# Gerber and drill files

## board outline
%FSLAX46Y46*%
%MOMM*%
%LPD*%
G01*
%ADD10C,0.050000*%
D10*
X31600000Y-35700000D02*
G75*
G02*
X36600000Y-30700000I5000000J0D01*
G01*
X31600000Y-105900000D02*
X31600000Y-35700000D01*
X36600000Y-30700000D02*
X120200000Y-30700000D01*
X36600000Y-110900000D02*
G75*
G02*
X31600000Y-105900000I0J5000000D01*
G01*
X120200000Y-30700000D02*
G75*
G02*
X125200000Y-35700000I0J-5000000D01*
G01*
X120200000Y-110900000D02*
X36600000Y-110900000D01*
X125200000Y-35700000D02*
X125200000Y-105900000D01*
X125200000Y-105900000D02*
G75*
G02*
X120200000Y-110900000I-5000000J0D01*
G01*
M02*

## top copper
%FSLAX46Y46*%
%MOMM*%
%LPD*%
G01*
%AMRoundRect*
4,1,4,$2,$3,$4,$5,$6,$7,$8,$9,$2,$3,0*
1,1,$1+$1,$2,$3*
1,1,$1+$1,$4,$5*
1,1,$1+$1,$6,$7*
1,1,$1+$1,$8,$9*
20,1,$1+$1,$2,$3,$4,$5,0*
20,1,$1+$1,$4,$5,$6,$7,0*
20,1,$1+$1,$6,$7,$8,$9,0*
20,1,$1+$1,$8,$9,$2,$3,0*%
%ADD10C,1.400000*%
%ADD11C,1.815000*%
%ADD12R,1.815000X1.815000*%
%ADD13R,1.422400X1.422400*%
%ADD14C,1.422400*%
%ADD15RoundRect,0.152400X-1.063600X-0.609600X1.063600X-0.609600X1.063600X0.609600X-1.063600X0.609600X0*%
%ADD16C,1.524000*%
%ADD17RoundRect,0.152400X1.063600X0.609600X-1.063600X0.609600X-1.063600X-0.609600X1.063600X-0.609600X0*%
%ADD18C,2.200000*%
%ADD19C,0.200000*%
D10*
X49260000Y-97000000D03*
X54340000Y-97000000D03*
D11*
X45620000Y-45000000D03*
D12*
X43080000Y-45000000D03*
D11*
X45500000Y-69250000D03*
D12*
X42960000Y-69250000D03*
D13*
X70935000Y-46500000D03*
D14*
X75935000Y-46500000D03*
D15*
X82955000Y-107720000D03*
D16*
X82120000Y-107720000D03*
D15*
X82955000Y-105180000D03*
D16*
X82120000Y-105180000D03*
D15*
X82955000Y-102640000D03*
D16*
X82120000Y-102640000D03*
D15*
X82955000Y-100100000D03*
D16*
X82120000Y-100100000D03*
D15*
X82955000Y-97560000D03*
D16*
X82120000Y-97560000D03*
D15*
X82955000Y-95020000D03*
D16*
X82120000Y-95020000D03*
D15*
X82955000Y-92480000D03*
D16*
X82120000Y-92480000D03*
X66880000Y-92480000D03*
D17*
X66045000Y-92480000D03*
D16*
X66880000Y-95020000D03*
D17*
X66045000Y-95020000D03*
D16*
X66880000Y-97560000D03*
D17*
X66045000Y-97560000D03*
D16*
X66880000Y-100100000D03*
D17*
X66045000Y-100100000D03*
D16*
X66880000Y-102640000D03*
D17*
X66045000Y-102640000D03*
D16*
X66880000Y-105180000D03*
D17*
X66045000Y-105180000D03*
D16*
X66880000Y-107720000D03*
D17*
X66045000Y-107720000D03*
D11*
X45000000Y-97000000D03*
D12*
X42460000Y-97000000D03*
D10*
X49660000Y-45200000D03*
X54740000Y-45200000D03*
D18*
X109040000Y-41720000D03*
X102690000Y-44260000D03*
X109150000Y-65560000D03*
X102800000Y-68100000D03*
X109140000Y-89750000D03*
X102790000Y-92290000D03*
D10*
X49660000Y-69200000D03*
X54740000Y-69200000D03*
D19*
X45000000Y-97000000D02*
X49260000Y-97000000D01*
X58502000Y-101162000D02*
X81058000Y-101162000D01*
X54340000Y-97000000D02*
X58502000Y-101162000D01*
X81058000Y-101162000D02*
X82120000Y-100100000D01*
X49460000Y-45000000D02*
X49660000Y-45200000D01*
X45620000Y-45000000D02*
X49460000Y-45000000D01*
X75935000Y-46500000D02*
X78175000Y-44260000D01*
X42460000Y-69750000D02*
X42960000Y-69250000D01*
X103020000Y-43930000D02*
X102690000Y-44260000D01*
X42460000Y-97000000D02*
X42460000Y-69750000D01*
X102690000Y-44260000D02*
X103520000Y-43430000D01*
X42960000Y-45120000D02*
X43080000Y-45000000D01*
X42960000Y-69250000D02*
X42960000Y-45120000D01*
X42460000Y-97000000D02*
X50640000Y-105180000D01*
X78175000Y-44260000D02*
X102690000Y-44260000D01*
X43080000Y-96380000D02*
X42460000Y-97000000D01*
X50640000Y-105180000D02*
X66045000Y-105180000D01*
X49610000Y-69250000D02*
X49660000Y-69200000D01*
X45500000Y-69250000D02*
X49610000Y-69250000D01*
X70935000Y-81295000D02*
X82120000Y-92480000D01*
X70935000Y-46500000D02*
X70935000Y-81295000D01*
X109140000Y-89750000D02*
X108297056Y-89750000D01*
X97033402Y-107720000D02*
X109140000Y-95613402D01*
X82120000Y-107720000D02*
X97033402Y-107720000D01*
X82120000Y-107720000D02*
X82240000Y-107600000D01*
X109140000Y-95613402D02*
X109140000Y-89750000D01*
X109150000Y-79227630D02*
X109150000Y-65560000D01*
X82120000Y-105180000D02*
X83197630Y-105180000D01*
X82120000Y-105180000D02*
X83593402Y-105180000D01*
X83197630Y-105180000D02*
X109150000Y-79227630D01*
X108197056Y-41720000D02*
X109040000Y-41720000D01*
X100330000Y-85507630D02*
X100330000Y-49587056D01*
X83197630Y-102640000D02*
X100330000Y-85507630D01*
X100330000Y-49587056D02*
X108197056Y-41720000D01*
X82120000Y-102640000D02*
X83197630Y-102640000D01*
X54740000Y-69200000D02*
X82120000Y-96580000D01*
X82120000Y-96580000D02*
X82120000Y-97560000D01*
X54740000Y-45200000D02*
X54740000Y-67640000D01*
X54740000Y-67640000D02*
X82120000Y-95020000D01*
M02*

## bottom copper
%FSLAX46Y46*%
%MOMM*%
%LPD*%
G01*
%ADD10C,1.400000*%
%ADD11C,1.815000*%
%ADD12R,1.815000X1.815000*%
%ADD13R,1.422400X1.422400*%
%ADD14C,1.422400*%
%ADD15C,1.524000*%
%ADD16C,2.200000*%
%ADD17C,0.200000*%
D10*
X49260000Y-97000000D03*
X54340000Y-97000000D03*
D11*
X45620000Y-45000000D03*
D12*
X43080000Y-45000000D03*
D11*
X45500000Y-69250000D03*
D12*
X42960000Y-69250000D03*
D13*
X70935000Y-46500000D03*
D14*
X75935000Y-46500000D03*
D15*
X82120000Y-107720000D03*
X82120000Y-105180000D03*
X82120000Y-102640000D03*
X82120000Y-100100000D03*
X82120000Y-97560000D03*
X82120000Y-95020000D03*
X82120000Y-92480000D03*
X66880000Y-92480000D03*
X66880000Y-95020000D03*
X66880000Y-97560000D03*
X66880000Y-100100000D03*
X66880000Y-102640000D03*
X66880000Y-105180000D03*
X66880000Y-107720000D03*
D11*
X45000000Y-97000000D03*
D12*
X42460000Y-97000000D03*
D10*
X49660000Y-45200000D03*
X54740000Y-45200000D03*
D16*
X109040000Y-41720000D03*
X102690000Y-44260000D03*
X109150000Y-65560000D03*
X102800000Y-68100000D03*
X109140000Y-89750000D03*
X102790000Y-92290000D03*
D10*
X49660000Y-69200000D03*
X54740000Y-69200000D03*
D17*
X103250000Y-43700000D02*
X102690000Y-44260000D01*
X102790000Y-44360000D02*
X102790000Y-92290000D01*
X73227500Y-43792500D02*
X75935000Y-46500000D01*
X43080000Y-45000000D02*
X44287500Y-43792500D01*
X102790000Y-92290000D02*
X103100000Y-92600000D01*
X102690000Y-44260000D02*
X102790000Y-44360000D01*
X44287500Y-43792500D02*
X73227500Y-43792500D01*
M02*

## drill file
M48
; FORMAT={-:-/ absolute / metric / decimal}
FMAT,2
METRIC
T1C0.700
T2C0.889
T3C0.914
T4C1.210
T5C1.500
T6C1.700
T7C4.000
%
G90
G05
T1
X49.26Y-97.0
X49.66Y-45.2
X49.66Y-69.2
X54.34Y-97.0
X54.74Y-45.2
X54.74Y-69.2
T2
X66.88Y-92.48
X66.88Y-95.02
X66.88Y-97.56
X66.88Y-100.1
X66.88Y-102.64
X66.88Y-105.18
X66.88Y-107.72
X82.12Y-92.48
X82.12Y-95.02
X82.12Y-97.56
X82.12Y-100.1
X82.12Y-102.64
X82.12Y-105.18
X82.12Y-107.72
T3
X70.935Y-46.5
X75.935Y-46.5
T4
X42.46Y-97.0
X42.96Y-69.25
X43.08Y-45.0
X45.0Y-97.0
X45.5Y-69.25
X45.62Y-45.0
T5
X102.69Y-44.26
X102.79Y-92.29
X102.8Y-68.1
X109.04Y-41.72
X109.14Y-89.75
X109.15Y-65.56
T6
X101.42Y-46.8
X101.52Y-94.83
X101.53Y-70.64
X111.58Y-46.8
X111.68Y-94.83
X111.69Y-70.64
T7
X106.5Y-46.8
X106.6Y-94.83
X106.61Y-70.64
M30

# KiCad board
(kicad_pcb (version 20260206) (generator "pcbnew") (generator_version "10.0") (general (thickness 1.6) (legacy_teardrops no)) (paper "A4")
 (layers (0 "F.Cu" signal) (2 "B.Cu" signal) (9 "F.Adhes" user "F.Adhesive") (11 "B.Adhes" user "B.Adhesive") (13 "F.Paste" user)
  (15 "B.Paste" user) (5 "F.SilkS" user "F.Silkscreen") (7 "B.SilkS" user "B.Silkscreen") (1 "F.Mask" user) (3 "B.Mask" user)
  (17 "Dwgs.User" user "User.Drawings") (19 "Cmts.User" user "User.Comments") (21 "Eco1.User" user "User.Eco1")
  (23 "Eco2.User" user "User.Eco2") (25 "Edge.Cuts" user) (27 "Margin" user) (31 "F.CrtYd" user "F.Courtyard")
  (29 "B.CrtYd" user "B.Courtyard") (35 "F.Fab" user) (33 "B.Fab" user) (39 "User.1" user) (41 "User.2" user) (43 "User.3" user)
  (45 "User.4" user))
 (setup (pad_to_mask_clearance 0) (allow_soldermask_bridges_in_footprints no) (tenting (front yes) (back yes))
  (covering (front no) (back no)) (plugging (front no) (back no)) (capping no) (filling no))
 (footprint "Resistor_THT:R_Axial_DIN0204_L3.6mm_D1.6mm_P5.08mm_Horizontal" (layer "F.Cu") (at 49.26 97)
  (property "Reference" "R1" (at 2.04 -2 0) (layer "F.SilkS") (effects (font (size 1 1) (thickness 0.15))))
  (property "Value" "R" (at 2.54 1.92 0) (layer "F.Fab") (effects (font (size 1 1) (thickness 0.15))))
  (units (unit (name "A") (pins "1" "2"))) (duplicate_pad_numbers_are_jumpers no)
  (pad "1" thru_hole circle (at 0 0) (size 1.4 1.4) (drill 0.7) (layers "*.Cu" "*.Mask") (remove_unused_layers no) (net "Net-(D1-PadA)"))
  (pad "2" thru_hole circle (at 5.08 0) (size 1.4 1.4) (drill 0.7) (layers "*.Cu" "*.Mask") (remove_unused_layers no) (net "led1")))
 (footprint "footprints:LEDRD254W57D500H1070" (layer "F.Cu") (at 44.35 45)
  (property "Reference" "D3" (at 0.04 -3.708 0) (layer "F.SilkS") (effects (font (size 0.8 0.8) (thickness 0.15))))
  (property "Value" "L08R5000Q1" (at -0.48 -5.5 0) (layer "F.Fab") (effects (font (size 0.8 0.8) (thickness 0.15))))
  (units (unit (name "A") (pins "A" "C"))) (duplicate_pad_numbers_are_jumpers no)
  (pad "A" thru_hole circle (at 1.27 0) (size 1.815 1.815) (drill 1.21) (layers "*.Cu" "*.Mask") (remove_unused_layers no)
   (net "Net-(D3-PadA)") (solder_mask_margin 0.102))
  (pad "C" thru_hole rect (at -1.27 0) (size 1.815 1.815) (drill 1.21) (layers "*.Cu" "*.Mask") (remove_unused_layers no) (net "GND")
   (solder_mask_margin 0.102)))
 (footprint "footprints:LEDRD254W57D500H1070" (layer "F.Cu") (at 44.23 69.25)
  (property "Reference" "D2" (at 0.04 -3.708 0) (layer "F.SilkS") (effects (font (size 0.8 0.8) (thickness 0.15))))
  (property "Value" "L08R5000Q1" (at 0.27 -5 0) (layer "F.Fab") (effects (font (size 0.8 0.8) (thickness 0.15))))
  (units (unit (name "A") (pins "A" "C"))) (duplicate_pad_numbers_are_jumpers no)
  (pad "A" thru_hole circle (at 1.27 0) (size 1.815 1.815) (drill 1.21) (layers "*.Cu" "*.Mask") (remove_unused_layers no)
   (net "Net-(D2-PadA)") (solder_mask_margin 0.102))
  (pad "C" thru_hole rect (at -1.27 0) (size 1.815 1.815) (drill 1.21) (layers "*.Cu" "*.Mask") (remove_unused_layers no) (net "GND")
   (solder_mask_margin 0.102)))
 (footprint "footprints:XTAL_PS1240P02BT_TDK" (layer "F.Cu") (at 70.935 46.5)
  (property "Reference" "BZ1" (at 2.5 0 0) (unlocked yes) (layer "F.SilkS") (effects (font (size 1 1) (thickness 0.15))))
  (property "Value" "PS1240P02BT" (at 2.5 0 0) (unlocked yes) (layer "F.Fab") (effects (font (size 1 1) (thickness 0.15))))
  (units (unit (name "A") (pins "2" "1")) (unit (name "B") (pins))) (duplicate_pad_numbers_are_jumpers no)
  (pad "1" thru_hole rect (at 0 0) (size 1.4224 1.4224) (drill 0.9144) (layers "*.Cu" "*.Mask") (remove_unused_layers no) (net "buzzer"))
  (pad "2" thru_hole circle (at 5 0) (size 1.4224 1.4224) (drill 0.9144) (layers "*.Cu" "*.Mask") (remove_unused_layers no) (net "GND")))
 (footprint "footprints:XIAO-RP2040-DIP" (layer "F.Cu") (at 74.5 100.1 -90)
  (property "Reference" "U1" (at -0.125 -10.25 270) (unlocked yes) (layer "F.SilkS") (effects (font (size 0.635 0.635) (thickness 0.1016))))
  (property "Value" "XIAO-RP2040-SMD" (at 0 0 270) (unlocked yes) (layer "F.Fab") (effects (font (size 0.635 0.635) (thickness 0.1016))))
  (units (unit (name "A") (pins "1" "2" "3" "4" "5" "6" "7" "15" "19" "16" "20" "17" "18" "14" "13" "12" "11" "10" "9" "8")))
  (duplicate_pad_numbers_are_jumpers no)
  (pad "1" smd roundrect (at 7.62 -8.455) (size 2.432 1.524) (layers "F.Cu" "F.Mask") (roundrect_rratio 0.1) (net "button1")
   (thermal_bridge_angle 45))
  (pad "1" thru_hole circle (at 7.62 -7.62) (size 1.524 1.524) (drill 0.889) (layers "*.Cu" "*.Mask") (remove_unused_layers no)
   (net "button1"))
  (pad "2" smd roundrect (at 5.08 -8.455) (size 2.432 1.524) (layers "F.Cu" "F.Mask") (roundrect_rratio 0.1) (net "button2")
   (thermal_bridge_angle 45))
  (pad "2" thru_hole circle (at 5.08 -7.62) (size 1.524 1.524) (drill 0.889) (layers "*.Cu" "*.Mask") (remove_unused_layers no)
   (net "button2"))
  (pad "3" smd roundrect (at 2.54 -8.455) (size 2.432 1.524) (layers "F.Cu" "F.Mask") (roundrect_rratio 0.1) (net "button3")
   (thermal_bridge_angle 45))
  (pad "3" thru_hole circle (at 2.54 -7.62) (size 1.524 1.524) (drill 0.889) (layers "*.Cu" "*.Mask") (remove_unused_layers no)
   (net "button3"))
  (pad "4" smd roundrect (at 0 -8.455) (size 2.432 1.524) (layers "F.Cu" "F.Mask") (roundrect_rratio 0.1) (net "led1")
   (thermal_bridge_angle 45))
  (pad "4" thru_hole circle (at 0 -7.62) (size 1.524 1.524) (drill 0.889) (layers "*.Cu" "*.Mask") (remove_unused_layers no) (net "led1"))
  (pad "5" smd roundrect (at -2.54 -8.455) (size 2.432 1.524) (layers "F.Cu" "F.Mask") (roundrect_rratio 0.1) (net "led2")
   (thermal_bridge_angle 45))
  (pad "5" thru_hole circle (at -2.54 -7.62) (size 1.524 1.524) (drill 0.889) (layers "*.Cu" "*.Mask") (remove_unused_layers no)
   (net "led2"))
  (pad "6" smd roundrect (at -5.08 -8.455) (size 2.432 1.524) (layers "F.Cu" "F.Mask") (roundrect_rratio 0.1) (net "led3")
   (thermal_bridge_angle 45))
  (pad "6" thru_hole circle (at -5.08 -7.62) (size 1.524 1.524) (drill 0.889) (layers "*.Cu" "*.Mask") (remove_unused_layers no)
   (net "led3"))
  (pad "7" smd roundrect (at -7.62 -8.455) (size 2.432 1.524) (layers "F.Cu" "F.Mask") (roundrect_rratio 0.1) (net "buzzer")
   (thermal_bridge_angle 45))
  (pad "7" thru_hole circle (at -7.62 -7.62) (size 1.524 1.524) (drill 0.889) (layers "*.Cu" "*.Mask") (remove_unused_layers no)
   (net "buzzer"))
  (pad "8" thru_hole circle (at -7.62 7.62 180) (size 1.524 1.524) (drill 0.889) (layers "*.Cu" "*.Mask") (remove_unused_layers no)
   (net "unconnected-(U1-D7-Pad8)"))
  (pad "8" smd roundrect (at -7.62 8.455 180) (size 2.432 1.524) (layers "F.Cu" "F.Mask") (roundrect_rratio 0.1)
   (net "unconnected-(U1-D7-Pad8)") (thermal_bridge_angle 45))
  (pad "9" thru_hole circle (at -5.08 7.62 180) (size 1.524 1.524) (drill 0.889) (layers "*.Cu" "*.Mask") (remove_unused_layers no)
   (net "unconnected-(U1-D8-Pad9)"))
  (pad "9" smd roundrect (at -5.08 8.455 180) (size 2.432 1.524) (layers "F.Cu" "F.Mask") (roundrect_rratio 0.1)
   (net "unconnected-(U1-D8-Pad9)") (thermal_bridge_angle 45))
  (pad "10" thru_hole circle (at -2.54 7.62 180) (size 1.524 1.524) (drill 0.889) (layers "*.Cu" "*.Mask") (remove_unused_layers no)
   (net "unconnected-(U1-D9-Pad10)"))
  (pad "10" smd roundrect (at -2.54 8.455 180) (size 2.432 1.524) (layers "F.Cu" "F.Mask") (roundrect_rratio 0.1)
   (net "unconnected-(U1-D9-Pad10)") (thermal_bridge_angle 45))
  (pad "11" thru_hole circle (at 0 7.62 180) (size 1.524 1.524) (drill 0.889) (layers "*.Cu" "*.Mask") (remove_unused_layers no)
   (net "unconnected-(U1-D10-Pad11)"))
  (pad "11" smd roundrect (at 0 8.455 180) (size 2.432 1.524) (layers "F.Cu" "F.Mask") (roundrect_rratio 0.1)
   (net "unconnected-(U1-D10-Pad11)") (thermal_bridge_angle 45))
  (pad "12" thru_hole circle (at 2.54 7.62 180) (size 1.524 1.524) (drill 0.889) (layers "*.Cu" "*.Mask") (remove_unused_layers no)
   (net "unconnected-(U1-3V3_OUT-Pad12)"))
  (pad "12" smd roundrect (at 2.54 8.455 180) (size 2.432 1.524) (layers "F.Cu" "F.Mask") (roundrect_rratio 0.1)
   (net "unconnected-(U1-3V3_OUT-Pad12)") (thermal_bridge_angle 45))
  (pad "13" thru_hole circle (at 5.08 7.62 180) (size 1.524 1.524) (drill 0.889) (layers "*.Cu" "*.Mask") (remove_unused_layers no)
   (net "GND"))
  (pad "13" smd roundrect (at 5.08 8.455 180) (size 2.432 1.524) (layers "F.Cu" "F.Mask") (roundrect_rratio 0.1) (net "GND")
   (thermal_bridge_angle 45))
  (pad "14" thru_hole circle (at 7.62 7.62 180) (size 1.524 1.524) (drill 0.889) (layers "*.Cu" "*.Mask") (remove_unused_layers no)
   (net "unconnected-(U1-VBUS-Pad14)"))
  (pad "14" smd roundrect (at 7.62 8.455 180) (size 2.432 1.524) (layers "F.Cu" "F.Mask") (roundrect_rratio 0.1)
   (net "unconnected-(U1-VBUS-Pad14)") (thermal_bridge_angle 45)))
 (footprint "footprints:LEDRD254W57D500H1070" (layer "F.Cu") (at 43.73 97)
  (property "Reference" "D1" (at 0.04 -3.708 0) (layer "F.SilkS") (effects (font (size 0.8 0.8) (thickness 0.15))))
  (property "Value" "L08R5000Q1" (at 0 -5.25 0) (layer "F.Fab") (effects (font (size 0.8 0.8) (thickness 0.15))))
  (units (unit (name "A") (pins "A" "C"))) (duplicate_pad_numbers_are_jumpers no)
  (pad "A" thru_hole circle (at 1.27 0) (size 1.815 1.815) (drill 1.21) (layers "*.Cu" "*.Mask") (remove_unused_layers no)
   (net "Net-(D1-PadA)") (solder_mask_margin 0.102))
  (pad "C" thru_hole rect (at -1.27 0) (size 1.815 1.815) (drill 1.21) (layers "*.Cu" "*.Mask") (remove_unused_layers no) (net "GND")
   (solder_mask_margin 0.102)))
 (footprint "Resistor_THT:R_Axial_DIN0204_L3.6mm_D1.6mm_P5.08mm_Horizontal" (layer "F.Cu") (at 49.66 45.2)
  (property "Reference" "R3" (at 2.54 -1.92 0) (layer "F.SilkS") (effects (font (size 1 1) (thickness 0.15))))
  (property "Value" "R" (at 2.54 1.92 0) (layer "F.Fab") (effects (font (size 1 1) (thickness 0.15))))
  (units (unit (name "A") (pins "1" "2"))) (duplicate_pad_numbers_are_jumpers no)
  (pad "1" thru_hole circle (at 0 0) (size 1.4 1.4) (drill 0.7) (layers "*.Cu" "*.Mask") (remove_unused_layers no) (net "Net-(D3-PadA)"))
  (pad "2" thru_hole circle (at 5.08 0) (size 1.4 1.4) (drill 0.7) (layers "*.Cu" "*.Mask") (remove_unused_layers no) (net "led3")))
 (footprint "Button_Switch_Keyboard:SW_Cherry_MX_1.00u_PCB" (layer "F.Cu") (at 109.04 41.72)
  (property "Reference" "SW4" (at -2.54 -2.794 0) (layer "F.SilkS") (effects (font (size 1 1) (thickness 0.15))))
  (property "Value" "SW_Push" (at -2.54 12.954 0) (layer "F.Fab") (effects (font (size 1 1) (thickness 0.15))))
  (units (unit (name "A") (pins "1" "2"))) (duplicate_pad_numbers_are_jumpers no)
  (pad "" np_thru_hole circle (at -7.62 5.08) (size 1.7 1.7) (drill 1.7) (layers "*.Cu" "*.Mask"))
  (pad "" np_thru_hole circle (at -2.54 5.08) (size 4 4) (drill 4) (layers "*.Cu" "*.Mask"))
  (pad "" np_thru_hole circle (at 2.54 5.08) (size 1.7 1.7) (drill 1.7) (layers "*.Cu" "*.Mask"))
  (pad "1" thru_hole circle (at 0 0) (size 2.2 2.2) (drill 1.5) (layers "*.Cu" "*.Mask") (remove_unused_layers no) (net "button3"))
  (pad "2" thru_hole circle (at -6.35 2.54) (size 2.2 2.2) (drill 1.5) (layers "*.Cu" "*.Mask") (remove_unused_layers no) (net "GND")))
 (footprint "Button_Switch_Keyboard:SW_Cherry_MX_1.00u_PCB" (layer "F.Cu") (at 109.15 65.56)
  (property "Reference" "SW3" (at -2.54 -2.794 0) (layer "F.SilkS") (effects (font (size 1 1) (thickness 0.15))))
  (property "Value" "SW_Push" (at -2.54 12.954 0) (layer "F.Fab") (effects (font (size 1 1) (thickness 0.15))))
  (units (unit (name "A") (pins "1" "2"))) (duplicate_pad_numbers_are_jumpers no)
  (pad "" np_thru_hole circle (at -7.62 5.08) (size 1.7 1.7) (drill 1.7) (layers "*.Cu" "*.Mask"))
  (pad "" np_thru_hole circle (at -2.54 5.08) (size 4 4) (drill 4) (layers "*.Cu" "*.Mask"))
  (pad "" np_thru_hole circle (at 2.54 5.08) (size 1.7 1.7) (drill 1.7) (layers "*.Cu" "*.Mask"))
  (pad "1" thru_hole circle (at 0 0) (size 2.2 2.2) (drill 1.5) (layers "*.Cu" "*.Mask") (remove_unused_layers no) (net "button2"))
  (pad "2" thru_hole circle (at -6.35 2.54) (size 2.2 2.2) (drill 1.5) (layers "*.Cu" "*.Mask") (remove_unused_layers no) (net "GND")))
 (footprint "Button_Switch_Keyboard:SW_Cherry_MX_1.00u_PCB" (layer "F.Cu") (at 109.14 89.75)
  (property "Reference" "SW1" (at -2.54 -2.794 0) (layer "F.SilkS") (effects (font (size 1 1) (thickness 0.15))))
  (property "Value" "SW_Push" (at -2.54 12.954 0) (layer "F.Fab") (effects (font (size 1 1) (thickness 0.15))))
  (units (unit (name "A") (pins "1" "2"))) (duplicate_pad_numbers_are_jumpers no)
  (pad "" np_thru_hole circle (at -7.62 5.08) (size 1.7 1.7) (drill 1.7) (layers "*.Cu" "*.Mask"))
  (pad "" np_thru_hole circle (at -2.54 5.08) (size 4 4) (drill 4) (layers "*.Cu" "*.Mask"))
  (pad "" np_thru_hole circle (at 2.54 5.08) (size 1.7 1.7) (drill 1.7) (layers "*.Cu" "*.Mask"))
  (pad "1" thru_hole circle (at 0 0) (size 2.2 2.2) (drill 1.5) (layers "*.Cu" "*.Mask") (remove_unused_layers no) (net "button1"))
  (pad "2" thru_hole circle (at -6.35 2.54) (size 2.2 2.2) (drill 1.5) (layers "*.Cu" "*.Mask") (remove_unused_layers no) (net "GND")))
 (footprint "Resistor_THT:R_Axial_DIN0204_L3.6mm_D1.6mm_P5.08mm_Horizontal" (layer "F.Cu") (at 49.66 69.2)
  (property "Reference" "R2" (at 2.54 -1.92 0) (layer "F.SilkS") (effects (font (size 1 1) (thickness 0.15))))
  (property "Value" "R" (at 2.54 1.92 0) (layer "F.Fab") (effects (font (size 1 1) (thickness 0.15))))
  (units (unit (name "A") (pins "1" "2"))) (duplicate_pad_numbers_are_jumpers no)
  (pad "1" thru_hole circle (at 0 0) (size 1.4 1.4) (drill 0.7) (layers "*.Cu" "*.Mask") (remove_unused_layers no) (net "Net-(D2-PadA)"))
  (pad "2" thru_hole circle (at 5.08 0) (size 1.4 1.4) (drill 0.7) (layers "*.Cu" "*.Mask") (remove_unused_layers no) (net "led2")))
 (gr_arc (start 31.6 35.7) (mid 33.064466 32.164466) (end 36.6 30.7) (stroke (width 0.05) (type default)) (layer "Edge.Cuts"))
 (gr_line (start 31.6 105.9) (end 31.6 35.7) (stroke (width 0.05) (type default)) (layer "Edge.Cuts"))
 (gr_line (start 36.6 30.7) (end 120.2 30.7) (stroke (width 0.05) (type default)) (layer "Edge.Cuts"))
 (gr_arc (start 36.6 110.9) (mid 33.064466 109.435534) (end 31.6 105.9) (stroke (width 0.05) (type default)) (layer "Edge.Cuts"))
 (gr_arc (start 120.2 30.7) (mid 123.735534 32.164466) (end 125.2 35.7) (stroke (width 0.05) (type default)) (layer "Edge.Cuts"))
 (gr_line (start 120.2 110.9) (end 36.6 110.9) (stroke (width 0.05) (type default)) (layer "Edge.Cuts"))
 (gr_line (start 125.2 35.7) (end 125.2 105.9) (stroke (width 0.05) (type default)) (layer "Edge.Cuts"))
 (gr_arc (start 125.2 105.9) (mid 123.735534 109.435534) (end 120.2 110.9) (stroke (width 0.05) (type default)) (layer "Edge.Cuts"))
 (segment (start 45 97) (end 49.26 97) (width 0.2) (layer "F.Cu") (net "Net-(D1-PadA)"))
 (segment (start 58.502 101.162) (end 81.058 101.162) (width 0.2) (layer "F.Cu") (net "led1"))
 (segment (start 54.34 97) (end 58.502 101.162) (width 0.2) (layer "F.Cu") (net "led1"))
 (segment (start 81.058 101.162) (end 82.12 100.1) (width 0.2) (layer "F.Cu") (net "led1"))
 (segment (start 49.46 45) (end 49.66 45.2) (width 0.2) (layer "F.Cu") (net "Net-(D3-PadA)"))
 (segment (start 45.62 45) (end 49.46 45) (width 0.2) (layer "F.Cu") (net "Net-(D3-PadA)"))
 (segment (start 75.935 46.5) (end 78.175 44.26) (width 0.2) (layer "F.Cu") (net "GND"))
 (segment (start 42.46 69.75) (end 42.96 69.25) (width 0.2) (layer "F.Cu") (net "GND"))
 (segment (start 103.02 43.93) (end 102.69 44.26) (width 0.2) (layer "F.Cu") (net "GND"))
 (segment (start 42.46 97) (end 42.46 69.75) (width 0.2) (layer "F.Cu") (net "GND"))
 (segment (start 102.69 44.26) (end 103.52 43.43) (width 0.2) (layer "F.Cu") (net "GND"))
 (segment (start 42.96 45.12) (end 43.08 45) (width 0.2) (layer "F.Cu") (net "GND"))
 (segment (start 42.96 69.25) (end 42.96 45.12) (width 0.2) (layer "F.Cu") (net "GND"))
 (segment (start 42.46 97) (end 50.64 105.18) (width 0.2) (layer "F.Cu") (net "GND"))
 (segment (start 78.175 44.26) (end 102.69 44.26) (width 0.2) (layer "F.Cu") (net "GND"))
 (segment (start 43.08 96.38) (end 42.46 97) (width 0.2) (layer "F.Cu") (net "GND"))
 (segment (start 50.64 105.18) (end 66.045 105.18) (width 0.2) (layer "F.Cu") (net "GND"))
 (segment (start 103.25 43.7) (end 102.69 44.26) (width 0.2) (layer "B.Cu") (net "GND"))
 (segment (start 102.79 44.36) (end 102.79 92.29) (width 0.2) (layer "B.Cu") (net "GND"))
 (segment (start 73.2275 43.7925) (end 75.935 46.5) (width 0.2) (layer "B.Cu") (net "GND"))
 (segment (start 43.08 45) (end 44.2875 43.7925) (width 0.2) (layer "B.Cu") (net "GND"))
 (segment (start 102.79 92.29) (end 103.1 92.6) (width 0.2) (layer "B.Cu") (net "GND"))
 (segment (start 102.69 44.26) (end 102.79 44.36) (width 0.2) (layer "B.Cu") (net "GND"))
 (segment (start 44.2875 43.7925) (end 73.2275 43.7925) (width 0.2) (layer "B.Cu") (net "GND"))
 (segment (start 49.61 69.25) (end 49.66 69.2) (width 0.2) (layer "F.Cu") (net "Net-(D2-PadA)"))
 (segment (start 45.5 69.25) (end 49.61 69.25) (width 0.2) (layer "F.Cu") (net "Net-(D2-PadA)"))
 (segment (start 70.935 81.295) (end 82.12 92.48) (width 0.2) (layer "F.Cu") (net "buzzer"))
 (segment (start 70.935 46.5) (end 70.935 81.295) (width 0.2) (layer "F.Cu") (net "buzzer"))
 (segment (start 109.14 89.75) (end 108.297056 89.75) (width 0.2) (layer "F.Cu") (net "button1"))
 (segment (start 97.033402 107.72) (end 109.14 95.613402) (width 0.2) (layer "F.Cu") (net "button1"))
 (segment (start 82.12 107.72) (end 97.033402 107.72) (width 0.2) (layer "F.Cu") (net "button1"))
 (segment (start 82.12 107.72) (end 82.24 107.6) (width 0.2) (layer "F.Cu") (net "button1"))
 (segment (start 109.14 95.613402) (end 109.14 89.75) (width 0.2) (layer "F.Cu") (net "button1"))
 (segment (start 109.15 79.22763) (end 109.15 65.56) (width 0.2) (layer "F.Cu") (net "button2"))
 (segment (start 82.12 105.18) (end 83.19763 105.18) (width 0.2) (layer "F.Cu") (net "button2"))
 (segment (start 82.12 105.18) (end 83.593402 105.18) (width 0.2) (layer "F.Cu") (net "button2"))
 (segment (start 83.19763 105.18) (end 109.15 79.22763) (width 0.2) (layer "F.Cu") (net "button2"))
 (segment (start 108.197056 41.72) (end 109.04 41.72) (width 0.2) (layer "F.Cu") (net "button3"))
 (segment (start 100.33 85.50763) (end 100.33 49.587056) (width 0.2) (layer "F.Cu") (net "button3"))
 (segment (start 83.19763 102.64) (end 100.33 85.50763) (width 0.2) (layer "F.Cu") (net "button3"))
 (segment (start 100.33 49.587056) (end 108.197056 41.72) (width 0.2) (layer "F.Cu") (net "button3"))
 (segment (start 82.12 102.64) (end 83.19763 102.64) (width 0.2) (layer "F.Cu") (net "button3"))
 (segment (start 54.74 69.2) (end 82.12 96.58) (width 0.2) (layer "F.Cu") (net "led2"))
 (segment (start 82.12 96.58) (end 82.12 97.56) (width 0.2) (layer "F.Cu") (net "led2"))
 (segment (start 54.74 45.2) (end 54.74 67.64) (width 0.2) (layer "F.Cu") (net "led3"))
 (segment (start 54.74 67.64) (end 82.12 95.02) (width 0.2) (layer "F.Cu") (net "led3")))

